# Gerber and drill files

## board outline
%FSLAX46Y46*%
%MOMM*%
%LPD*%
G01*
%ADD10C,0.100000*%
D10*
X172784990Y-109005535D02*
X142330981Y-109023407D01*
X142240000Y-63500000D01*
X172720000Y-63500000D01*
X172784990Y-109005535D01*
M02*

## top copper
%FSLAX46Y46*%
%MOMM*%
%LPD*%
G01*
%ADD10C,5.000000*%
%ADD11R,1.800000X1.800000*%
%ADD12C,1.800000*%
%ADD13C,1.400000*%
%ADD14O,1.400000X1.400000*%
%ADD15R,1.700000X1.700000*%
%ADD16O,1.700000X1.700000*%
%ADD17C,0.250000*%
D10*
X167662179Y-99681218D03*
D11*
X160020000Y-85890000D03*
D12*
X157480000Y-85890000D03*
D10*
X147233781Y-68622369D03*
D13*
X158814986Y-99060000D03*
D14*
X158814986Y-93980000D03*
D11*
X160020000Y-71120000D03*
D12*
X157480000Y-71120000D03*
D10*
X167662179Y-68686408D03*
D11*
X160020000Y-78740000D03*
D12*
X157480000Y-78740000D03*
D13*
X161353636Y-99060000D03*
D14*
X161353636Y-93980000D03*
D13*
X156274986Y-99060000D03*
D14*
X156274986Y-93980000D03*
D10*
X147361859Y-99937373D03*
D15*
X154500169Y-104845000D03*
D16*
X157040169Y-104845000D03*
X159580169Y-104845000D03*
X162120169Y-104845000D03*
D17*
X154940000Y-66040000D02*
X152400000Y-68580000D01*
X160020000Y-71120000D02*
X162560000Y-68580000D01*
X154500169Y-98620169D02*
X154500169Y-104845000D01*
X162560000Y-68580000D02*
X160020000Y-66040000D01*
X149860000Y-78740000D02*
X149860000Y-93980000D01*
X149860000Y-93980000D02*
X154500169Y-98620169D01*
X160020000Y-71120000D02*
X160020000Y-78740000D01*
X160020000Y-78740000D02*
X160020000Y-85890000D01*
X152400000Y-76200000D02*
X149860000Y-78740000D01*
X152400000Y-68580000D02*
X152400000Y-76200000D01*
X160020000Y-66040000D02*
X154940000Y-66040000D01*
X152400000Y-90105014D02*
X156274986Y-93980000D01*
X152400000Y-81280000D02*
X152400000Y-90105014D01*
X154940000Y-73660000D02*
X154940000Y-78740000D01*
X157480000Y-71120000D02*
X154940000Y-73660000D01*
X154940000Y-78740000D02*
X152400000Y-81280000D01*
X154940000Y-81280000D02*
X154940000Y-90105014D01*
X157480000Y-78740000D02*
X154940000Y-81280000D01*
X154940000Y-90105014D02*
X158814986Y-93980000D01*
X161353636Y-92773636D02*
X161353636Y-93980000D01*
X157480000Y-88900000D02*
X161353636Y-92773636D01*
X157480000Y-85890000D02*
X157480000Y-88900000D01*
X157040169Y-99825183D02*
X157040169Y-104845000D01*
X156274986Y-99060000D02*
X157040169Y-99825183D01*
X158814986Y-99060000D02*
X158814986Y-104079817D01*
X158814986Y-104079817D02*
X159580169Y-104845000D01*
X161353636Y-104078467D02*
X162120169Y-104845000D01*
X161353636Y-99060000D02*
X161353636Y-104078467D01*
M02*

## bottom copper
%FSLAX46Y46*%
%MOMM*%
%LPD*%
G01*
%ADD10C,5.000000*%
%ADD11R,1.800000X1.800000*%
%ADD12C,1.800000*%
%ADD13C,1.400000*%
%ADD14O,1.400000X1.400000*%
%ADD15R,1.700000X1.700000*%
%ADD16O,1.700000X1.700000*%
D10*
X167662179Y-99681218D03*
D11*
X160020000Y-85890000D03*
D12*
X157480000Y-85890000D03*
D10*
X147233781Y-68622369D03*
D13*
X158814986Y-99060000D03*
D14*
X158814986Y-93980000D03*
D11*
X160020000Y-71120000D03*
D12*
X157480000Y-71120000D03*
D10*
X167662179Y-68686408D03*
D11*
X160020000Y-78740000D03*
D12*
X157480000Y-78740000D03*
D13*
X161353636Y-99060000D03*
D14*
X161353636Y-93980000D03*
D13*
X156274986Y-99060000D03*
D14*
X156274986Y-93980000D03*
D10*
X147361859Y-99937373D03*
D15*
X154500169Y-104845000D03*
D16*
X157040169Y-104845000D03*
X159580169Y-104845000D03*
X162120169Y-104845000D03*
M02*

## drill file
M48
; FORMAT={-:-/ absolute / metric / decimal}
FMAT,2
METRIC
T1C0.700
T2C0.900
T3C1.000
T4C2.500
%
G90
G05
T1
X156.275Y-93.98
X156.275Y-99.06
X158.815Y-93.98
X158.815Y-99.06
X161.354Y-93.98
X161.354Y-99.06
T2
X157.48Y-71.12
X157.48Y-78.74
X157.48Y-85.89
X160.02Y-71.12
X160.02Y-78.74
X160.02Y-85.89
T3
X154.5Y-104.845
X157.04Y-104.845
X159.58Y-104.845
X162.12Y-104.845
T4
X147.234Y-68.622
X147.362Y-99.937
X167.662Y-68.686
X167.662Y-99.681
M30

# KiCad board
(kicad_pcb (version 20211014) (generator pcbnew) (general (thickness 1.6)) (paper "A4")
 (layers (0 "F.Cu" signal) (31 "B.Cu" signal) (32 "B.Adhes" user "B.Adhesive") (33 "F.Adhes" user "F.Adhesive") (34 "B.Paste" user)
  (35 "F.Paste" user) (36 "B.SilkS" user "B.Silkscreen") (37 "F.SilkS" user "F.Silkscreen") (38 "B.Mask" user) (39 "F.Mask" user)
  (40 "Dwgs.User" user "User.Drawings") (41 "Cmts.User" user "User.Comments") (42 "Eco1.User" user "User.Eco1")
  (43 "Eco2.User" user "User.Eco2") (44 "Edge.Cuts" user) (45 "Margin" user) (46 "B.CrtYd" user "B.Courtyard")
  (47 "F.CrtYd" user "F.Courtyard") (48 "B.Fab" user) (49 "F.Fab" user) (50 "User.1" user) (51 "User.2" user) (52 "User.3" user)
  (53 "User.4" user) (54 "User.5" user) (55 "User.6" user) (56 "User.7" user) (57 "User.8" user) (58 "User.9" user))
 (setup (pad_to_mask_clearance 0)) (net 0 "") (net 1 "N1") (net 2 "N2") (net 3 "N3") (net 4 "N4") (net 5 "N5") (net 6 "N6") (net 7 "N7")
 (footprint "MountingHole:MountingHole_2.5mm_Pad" (layer "F.Cu") (at 167.662179 99.681218)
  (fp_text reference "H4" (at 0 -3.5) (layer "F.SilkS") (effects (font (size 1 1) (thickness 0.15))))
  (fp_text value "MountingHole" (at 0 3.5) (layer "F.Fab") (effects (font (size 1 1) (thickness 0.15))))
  (pad "1" thru_hole circle (at 0 0) (size 5 5) (drill 2.5) (layers *.Cu *.Mask)))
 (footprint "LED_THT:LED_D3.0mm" (layer "F.Cu") (at 160.02 85.89 180)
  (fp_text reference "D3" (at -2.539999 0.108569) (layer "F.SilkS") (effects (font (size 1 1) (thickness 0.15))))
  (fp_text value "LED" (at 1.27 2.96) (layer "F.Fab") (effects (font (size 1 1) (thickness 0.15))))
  (pad "1" thru_hole rect (at 0 0 180) (size 1.8 1.8) (drill 0.9) (layers *.Cu *.Mask) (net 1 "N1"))
  (pad "2" thru_hole circle (at 2.54 0 180) (size 1.8 1.8) (drill 0.9) (layers *.Cu *.Mask) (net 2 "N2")))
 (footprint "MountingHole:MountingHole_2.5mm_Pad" (layer "F.Cu") (at 147.233781 68.622369)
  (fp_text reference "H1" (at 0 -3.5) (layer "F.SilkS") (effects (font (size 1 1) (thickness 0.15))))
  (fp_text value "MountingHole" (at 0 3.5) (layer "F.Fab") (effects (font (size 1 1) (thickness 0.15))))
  (pad "1" thru_hole circle (at 0 0) (size 5 5) (drill 2.5) (layers *.Cu *.Mask)))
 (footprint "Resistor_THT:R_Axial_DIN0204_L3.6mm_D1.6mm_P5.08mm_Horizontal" (layer "F.Cu") (at 158.814986 99.06 90)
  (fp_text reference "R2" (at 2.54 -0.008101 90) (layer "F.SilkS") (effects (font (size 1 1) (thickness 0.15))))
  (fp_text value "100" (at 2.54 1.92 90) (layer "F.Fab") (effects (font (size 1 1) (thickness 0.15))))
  (pad "1" thru_hole circle (at 0 0 90) (size 1.4 1.4) (drill 0.7) (layers *.Cu *.Mask) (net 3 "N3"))
  (pad "2" thru_hole oval (at 5.08 0 90) (size 1.4 1.4) (drill 0.7) (layers *.Cu *.Mask) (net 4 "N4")))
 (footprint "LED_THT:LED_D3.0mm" (layer "F.Cu") (at 160.02 71.12 180)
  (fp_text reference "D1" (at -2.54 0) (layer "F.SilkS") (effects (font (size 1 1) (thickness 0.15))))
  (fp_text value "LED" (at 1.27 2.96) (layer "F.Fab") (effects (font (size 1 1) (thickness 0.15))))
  (pad "1" thru_hole rect (at 0 0 180) (size 1.8 1.8) (drill 0.9) (layers *.Cu *.Mask) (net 1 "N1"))
  (pad "2" thru_hole circle (at 2.54 0 180) (size 1.8 1.8) (drill 0.9) (layers *.Cu *.Mask) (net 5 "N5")))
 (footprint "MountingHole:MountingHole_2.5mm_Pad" (layer "F.Cu") (at 167.662179 68.686408)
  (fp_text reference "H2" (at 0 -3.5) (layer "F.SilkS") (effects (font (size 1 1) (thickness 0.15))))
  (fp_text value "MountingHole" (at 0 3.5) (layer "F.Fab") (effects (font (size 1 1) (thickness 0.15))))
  (pad "1" thru_hole circle (at 0 0) (size 5 5) (drill 2.5) (layers *.Cu *.Mask)))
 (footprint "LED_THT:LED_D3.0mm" (layer "F.Cu") (at 160.02 78.74 180)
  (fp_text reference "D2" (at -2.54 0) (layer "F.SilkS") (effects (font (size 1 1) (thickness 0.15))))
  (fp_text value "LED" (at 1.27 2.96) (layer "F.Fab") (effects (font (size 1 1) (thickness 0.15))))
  (pad "1" thru_hole rect (at 0 0 180) (size 1.8 1.8) (drill 0.9) (layers *.Cu *.Mask) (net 1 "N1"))
  (pad "2" thru_hole circle (at 2.54 0 180) (size 1.8 1.8) (drill 0.9) (layers *.Cu *.Mask) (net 4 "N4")))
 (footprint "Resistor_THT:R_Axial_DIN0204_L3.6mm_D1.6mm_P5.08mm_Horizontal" (layer "F.Cu") (at 161.353636 99.06 90)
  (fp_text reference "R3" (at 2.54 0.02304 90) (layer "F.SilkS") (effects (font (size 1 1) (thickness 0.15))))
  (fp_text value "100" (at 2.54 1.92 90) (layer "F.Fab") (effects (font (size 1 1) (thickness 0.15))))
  (pad "1" thru_hole circle (at 0 0 90) (size 1.4 1.4) (drill 0.7) (layers *.Cu *.Mask) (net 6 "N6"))
  (pad "2" thru_hole oval (at 5.08 0 90) (size 1.4 1.4) (drill 0.7) (layers *.Cu *.Mask) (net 2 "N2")))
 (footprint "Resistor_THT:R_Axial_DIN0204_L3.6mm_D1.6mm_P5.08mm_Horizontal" (layer "F.Cu") (at 156.274986 99.06 90)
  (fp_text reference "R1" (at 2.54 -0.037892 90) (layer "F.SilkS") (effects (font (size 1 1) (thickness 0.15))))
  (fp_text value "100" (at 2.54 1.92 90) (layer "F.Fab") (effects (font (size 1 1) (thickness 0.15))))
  (pad "1" thru_hole circle (at 0 0 90) (size 1.4 1.4) (drill 0.7) (layers *.Cu *.Mask) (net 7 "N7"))
  (pad "2" thru_hole oval (at 5.08 0 90) (size 1.4 1.4) (drill 0.7) (layers *.Cu *.Mask) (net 5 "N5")))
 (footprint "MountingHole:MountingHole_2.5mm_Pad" (layer "F.Cu") (at 147.361859 99.937373)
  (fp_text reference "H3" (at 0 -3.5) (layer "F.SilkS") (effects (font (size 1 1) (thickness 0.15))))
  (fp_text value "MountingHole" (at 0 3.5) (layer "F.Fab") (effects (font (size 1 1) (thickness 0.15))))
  (pad "1" thru_hole circle (at 0 0) (size 5 5) (drill 2.5) (layers *.Cu *.Mask)))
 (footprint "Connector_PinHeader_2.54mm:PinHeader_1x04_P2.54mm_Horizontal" (layer "B.Cu") (at 154.500169 104.845 -90)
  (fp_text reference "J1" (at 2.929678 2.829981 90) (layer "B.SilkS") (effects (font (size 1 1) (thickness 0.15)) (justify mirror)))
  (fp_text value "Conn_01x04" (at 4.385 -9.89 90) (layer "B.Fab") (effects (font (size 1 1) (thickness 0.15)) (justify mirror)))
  (pad "1" thru_hole rect (at 0 0 270) (size 1.7 1.7) (drill 1) (layers *.Cu *.Mask) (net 1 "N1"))
  (pad "2" thru_hole oval (at 0 -2.54 270) (size 1.7 1.7) (drill 1) (layers *.Cu *.Mask) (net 7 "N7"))
  (pad "3" thru_hole oval (at 0 -5.08 270) (size 1.7 1.7) (drill 1) (layers *.Cu *.Mask) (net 3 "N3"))
  (pad "4" thru_hole oval (at 0 -7.62 270) (size 1.7 1.7) (drill 1) (layers *.Cu *.Mask) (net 6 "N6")))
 (gr_poly
  (pts (xy 172.78499 109.005535) (xy 142.330981 109.023407) (xy 142.24 63.5) (xy 172.72 63.5)) (layer "Edge.Cuts") (width 0.1) (fill none))
 (segment (start 154.94 66.04) (end 152.4 68.58) (width 0.25) (layer "F.Cu") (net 1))
 (segment (start 160.02 71.12) (end 162.56 68.58) (width 0.25) (layer "F.Cu") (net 1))
 (segment (start 154.500169 98.620169) (end 154.500169 104.845) (width 0.25) (layer "F.Cu") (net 1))
 (segment (start 162.56 68.58) (end 160.02 66.04) (width 0.25) (layer "F.Cu") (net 1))
 (segment (start 149.86 78.74) (end 149.86 93.98) (width 0.25) (layer "F.Cu") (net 1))
 (segment (start 149.86 93.98) (end 154.500169 98.620169) (width 0.25) (layer "F.Cu") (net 1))
 (segment (start 160.02 71.12) (end 160.02 78.74) (width 0.25) (layer "F.Cu") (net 1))
 (segment (start 160.02 78.74) (end 160.02 85.89) (width 0.25) (layer "F.Cu") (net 1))
 (segment (start 152.4 76.2) (end 149.86 78.74) (width 0.25) (layer "F.Cu") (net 1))
 (segment (start 152.4 68.58) (end 152.4 76.2) (width 0.25) (layer "F.Cu") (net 1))
 (segment (start 160.02 66.04) (end 154.94 66.04) (width 0.25) (layer "F.Cu") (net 1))
 (segment (start 152.4 90.105014) (end 156.274986 93.98) (width 0.25) (layer "F.Cu") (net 5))
 (segment (start 152.4 81.28) (end 152.4 90.105014) (width 0.25) (layer "F.Cu") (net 5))
 (segment (start 154.94 73.66) (end 154.94 78.74) (width 0.25) (layer "F.Cu") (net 5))
 (segment (start 157.48 71.12) (end 154.94 73.66) (width 0.25) (layer "F.Cu") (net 5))
 (segment (start 154.94 78.74) (end 152.4 81.28) (width 0.25) (layer "F.Cu") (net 5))
 (segment (start 154.94 81.28) (end 154.94 90.105014) (width 0.25) (layer "F.Cu") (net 4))
 (segment (start 157.48 78.74) (end 154.94 81.28) (width 0.25) (layer "F.Cu") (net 4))
 (segment (start 154.94 90.105014) (end 158.814986 93.98) (width 0.25) (layer "F.Cu") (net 4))
 (segment (start 161.353636 92.773636) (end 161.353636 93.98) (width 0.25) (layer "F.Cu") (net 2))
 (segment (start 157.48 88.9) (end 161.353636 92.773636) (width 0.25) (layer "F.Cu") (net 2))
 (segment (start 157.48 85.89) (end 157.48 88.9) (width 0.25) (layer "F.Cu") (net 2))
 (segment (start 157.040169 99.825183) (end 157.040169 104.845) (width 0.25) (layer "F.Cu") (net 7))
 (segment (start 156.274986 99.06) (end 157.040169 99.825183) (width 0.25) (layer "F.Cu") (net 7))
 (segment (start 158.814986 99.06) (end 158.814986 104.079817) (width 0.25) (layer "F.Cu") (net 3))
 (segment (start 158.814986 104.079817) (end 159.580169 104.845) (width 0.25) (layer "F.Cu") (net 3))
 (segment (start 161.353636 104.078467) (end 162.120169 104.845) (width 0.25) (layer "F.Cu") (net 6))
 (segment (start 161.353636 99.06) (end 161.353636 104.078467) (width 0.25) (layer "F.Cu") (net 6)))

